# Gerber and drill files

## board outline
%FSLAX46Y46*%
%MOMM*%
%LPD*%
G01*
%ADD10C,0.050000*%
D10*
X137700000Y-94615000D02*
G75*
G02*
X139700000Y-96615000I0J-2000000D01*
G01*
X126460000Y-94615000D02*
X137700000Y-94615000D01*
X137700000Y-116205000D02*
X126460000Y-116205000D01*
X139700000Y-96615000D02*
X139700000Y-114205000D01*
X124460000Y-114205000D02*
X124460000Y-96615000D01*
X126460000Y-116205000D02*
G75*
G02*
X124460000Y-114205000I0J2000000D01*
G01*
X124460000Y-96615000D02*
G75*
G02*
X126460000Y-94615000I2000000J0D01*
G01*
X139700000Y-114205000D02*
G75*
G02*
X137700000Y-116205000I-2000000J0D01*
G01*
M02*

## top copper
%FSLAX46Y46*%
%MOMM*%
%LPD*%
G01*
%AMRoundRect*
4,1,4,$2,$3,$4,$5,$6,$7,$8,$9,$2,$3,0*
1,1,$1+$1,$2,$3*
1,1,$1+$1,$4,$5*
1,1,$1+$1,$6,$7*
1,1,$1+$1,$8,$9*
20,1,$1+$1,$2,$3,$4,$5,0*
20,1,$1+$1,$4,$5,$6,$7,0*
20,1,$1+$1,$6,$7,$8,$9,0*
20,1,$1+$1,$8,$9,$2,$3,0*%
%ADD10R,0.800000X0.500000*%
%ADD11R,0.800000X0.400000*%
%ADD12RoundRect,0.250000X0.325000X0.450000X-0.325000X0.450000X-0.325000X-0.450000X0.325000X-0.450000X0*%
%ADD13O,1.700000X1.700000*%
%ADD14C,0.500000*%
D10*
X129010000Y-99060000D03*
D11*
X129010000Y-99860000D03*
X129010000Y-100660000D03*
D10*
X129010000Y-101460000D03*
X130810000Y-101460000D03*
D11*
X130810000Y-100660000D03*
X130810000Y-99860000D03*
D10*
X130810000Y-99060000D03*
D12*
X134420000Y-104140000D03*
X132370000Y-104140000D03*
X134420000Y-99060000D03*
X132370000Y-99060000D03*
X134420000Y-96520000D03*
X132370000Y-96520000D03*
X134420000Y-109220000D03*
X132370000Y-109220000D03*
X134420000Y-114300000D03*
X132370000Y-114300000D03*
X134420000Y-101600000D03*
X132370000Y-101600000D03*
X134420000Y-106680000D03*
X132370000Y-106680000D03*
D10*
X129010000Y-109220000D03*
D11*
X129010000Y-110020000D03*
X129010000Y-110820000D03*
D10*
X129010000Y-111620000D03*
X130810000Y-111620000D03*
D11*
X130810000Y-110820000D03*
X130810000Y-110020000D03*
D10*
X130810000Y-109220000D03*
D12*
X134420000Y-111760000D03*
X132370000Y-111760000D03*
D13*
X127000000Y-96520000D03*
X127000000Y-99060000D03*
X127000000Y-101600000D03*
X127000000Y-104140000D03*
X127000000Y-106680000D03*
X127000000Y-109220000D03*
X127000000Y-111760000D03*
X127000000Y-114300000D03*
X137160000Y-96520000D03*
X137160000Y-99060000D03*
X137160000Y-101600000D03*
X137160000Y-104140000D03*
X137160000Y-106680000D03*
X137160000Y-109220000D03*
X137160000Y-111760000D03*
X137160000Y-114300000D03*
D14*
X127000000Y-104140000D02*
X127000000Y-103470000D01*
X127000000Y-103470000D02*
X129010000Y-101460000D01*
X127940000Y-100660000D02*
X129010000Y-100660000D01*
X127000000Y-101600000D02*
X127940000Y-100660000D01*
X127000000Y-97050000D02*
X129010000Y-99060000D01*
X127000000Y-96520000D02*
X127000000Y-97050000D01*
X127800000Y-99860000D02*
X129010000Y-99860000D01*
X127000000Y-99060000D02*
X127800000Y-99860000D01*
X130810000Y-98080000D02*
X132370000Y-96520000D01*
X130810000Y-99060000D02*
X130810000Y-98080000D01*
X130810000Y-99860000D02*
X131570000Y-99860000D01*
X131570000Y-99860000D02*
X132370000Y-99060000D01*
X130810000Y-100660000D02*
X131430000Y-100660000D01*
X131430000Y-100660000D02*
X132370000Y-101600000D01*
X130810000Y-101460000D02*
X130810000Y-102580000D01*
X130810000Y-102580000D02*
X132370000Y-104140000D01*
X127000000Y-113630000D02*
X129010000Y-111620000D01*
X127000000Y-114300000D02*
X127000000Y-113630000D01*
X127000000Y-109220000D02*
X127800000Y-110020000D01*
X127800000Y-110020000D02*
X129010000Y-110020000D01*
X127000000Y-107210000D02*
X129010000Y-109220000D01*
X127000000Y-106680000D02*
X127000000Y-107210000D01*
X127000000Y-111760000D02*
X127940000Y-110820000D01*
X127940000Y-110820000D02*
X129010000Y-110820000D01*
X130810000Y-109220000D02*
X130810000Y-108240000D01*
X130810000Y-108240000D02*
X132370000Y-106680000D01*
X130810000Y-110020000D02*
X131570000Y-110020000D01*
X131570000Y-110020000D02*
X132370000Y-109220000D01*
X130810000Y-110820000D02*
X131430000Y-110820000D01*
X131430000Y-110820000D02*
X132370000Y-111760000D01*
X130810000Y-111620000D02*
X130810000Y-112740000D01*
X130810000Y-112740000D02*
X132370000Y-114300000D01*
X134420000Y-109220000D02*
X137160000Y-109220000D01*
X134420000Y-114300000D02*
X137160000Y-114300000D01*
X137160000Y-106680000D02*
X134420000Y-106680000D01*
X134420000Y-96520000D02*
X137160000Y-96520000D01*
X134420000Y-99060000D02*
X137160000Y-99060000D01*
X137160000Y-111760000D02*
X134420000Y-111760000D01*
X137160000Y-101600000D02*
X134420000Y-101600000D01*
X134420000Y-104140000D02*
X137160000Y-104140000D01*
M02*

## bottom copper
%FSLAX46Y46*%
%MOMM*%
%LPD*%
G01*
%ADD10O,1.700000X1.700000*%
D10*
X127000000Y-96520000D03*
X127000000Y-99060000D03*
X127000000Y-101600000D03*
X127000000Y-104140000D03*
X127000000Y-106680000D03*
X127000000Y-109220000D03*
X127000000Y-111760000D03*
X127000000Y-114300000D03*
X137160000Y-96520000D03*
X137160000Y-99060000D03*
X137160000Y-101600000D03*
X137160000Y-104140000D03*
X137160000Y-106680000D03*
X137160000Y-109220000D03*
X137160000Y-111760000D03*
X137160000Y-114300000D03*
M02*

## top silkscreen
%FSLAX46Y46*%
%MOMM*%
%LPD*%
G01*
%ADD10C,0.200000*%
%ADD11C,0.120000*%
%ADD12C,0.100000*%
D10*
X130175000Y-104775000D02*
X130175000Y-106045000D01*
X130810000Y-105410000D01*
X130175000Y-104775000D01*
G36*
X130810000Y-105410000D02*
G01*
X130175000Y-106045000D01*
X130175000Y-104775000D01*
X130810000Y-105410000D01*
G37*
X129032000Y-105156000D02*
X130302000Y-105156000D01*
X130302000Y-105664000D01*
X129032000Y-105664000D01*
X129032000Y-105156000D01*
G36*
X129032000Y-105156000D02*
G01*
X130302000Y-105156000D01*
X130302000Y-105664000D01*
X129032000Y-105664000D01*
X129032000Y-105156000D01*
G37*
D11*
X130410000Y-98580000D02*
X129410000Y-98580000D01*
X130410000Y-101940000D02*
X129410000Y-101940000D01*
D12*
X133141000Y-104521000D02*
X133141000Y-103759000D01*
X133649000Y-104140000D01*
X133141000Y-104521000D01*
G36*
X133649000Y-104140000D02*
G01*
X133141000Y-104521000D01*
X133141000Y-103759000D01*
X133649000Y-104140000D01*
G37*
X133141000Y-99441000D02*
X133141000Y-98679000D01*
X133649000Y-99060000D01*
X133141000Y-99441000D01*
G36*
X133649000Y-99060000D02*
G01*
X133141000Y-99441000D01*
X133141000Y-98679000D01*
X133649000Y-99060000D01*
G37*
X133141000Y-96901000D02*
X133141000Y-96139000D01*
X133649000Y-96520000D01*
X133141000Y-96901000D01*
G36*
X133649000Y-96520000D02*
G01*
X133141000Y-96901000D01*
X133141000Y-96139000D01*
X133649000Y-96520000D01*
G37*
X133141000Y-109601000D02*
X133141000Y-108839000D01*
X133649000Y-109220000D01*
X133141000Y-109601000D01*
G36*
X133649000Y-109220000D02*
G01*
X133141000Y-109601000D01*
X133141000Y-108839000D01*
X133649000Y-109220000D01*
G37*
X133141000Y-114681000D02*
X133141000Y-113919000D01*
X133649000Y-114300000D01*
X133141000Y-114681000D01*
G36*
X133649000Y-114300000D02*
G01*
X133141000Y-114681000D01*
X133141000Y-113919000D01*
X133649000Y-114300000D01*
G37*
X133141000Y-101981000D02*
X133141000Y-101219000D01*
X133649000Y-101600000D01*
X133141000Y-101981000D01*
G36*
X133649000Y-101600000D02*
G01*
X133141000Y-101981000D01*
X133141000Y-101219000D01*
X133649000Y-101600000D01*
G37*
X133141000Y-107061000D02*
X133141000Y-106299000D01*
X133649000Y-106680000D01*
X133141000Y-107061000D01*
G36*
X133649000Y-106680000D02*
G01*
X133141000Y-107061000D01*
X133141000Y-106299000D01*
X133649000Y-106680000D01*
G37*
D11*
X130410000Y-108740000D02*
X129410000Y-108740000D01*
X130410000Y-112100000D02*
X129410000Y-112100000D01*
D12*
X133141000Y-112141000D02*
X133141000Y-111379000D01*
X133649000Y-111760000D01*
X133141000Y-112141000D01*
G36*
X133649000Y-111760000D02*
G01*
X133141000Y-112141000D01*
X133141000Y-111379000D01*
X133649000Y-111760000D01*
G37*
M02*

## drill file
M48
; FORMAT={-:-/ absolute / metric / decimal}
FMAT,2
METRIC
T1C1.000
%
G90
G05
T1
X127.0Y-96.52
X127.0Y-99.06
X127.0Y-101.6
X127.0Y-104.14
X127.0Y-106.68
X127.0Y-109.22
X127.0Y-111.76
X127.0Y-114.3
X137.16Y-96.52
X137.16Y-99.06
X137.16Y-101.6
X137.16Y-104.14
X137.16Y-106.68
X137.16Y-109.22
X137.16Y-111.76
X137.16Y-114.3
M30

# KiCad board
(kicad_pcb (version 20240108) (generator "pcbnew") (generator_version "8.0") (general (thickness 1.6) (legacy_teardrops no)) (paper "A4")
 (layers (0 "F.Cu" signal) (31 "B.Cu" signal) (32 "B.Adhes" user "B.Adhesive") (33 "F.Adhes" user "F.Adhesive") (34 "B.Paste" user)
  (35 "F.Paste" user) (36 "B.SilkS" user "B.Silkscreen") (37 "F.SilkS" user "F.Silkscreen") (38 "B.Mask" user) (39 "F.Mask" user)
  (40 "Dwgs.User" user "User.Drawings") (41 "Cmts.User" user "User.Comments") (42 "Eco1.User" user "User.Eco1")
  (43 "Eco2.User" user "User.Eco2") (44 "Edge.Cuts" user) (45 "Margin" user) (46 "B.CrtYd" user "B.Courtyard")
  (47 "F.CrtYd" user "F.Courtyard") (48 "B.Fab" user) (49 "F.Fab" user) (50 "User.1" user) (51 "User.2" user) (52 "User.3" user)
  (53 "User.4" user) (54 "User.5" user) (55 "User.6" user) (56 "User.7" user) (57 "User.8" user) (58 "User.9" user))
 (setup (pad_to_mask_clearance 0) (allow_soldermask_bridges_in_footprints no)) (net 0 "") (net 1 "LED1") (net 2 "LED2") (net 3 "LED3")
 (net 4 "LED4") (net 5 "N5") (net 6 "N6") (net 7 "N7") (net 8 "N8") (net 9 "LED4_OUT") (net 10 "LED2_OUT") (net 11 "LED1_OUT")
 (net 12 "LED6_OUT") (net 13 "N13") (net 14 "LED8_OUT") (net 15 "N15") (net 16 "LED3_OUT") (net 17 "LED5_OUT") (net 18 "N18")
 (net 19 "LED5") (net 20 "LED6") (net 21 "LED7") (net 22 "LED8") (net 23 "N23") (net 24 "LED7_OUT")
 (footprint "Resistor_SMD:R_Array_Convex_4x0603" (layer "F.Cu") (at 129.91 100.26)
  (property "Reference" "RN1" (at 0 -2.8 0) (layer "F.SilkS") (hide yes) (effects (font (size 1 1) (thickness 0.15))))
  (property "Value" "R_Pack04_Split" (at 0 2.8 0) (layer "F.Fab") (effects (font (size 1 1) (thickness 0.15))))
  (fp_line (start 0.5 -1.68) (end -0.5 -1.68) (stroke (width 0.12) (type solid)) (layer "F.SilkS"))
  (fp_line (start 0.5 1.68) (end -0.5 1.68) (stroke (width 0.12) (type solid)) (layer "F.SilkS"))
  (pad "1" smd rect (at -0.9 -1.2) (size 0.8 0.5) (layers "F.Cu" "F.Paste" "F.Mask") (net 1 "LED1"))
  (pad "2" smd rect (at -0.9 -0.4) (size 0.8 0.4) (layers "F.Cu" "F.Paste" "F.Mask") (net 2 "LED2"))
  (pad "3" smd rect (at -0.9 0.4) (size 0.8 0.4) (layers "F.Cu" "F.Paste" "F.Mask") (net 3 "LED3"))
  (pad "4" smd rect (at -0.9 1.2) (size 0.8 0.5) (layers "F.Cu" "F.Paste" "F.Mask") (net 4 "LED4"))
  (pad "5" smd rect (at 0.9 1.2) (size 0.8 0.5) (layers "F.Cu" "F.Paste" "F.Mask") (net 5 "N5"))
  (pad "6" smd rect (at 0.9 0.4) (size 0.8 0.4) (layers "F.Cu" "F.Paste" "F.Mask") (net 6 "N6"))
  (pad "7" smd rect (at 0.9 -0.4) (size 0.8 0.4) (layers "F.Cu" "F.Paste" "F.Mask") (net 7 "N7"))
  (pad "8" smd rect (at 0.9 -1.2) (size 0.8 0.5) (layers "F.Cu" "F.Paste" "F.Mask") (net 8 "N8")))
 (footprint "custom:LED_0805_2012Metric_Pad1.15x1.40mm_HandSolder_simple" (layer "F.Cu") (at 133.395 104.14 180)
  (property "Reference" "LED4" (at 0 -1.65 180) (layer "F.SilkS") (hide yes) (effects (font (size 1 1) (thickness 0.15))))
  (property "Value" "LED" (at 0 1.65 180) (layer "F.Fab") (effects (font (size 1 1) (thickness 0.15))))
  (fp_poly (pts (xy 0.254 -0.381) (xy 0.254 0.381) (xy -0.254 0)) (stroke (width 0.1) (type solid)) (fill solid) (layer "F.SilkS"))
  (pad "1" smd roundrect (at -1.025 0 180) (size 1.15 1.4) (layers "F.Cu" "F.Paste" "F.Mask") (roundrect_rratio 0.217391) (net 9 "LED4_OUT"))
  (pad "2" smd roundrect (at 1.025 0 180) (size 1.15 1.4) (layers "F.Cu" "F.Paste" "F.Mask") (roundrect_rratio 0.217391) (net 5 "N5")))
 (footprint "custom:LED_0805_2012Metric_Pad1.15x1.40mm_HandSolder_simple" (layer "F.Cu") (at 133.395 99.06 180)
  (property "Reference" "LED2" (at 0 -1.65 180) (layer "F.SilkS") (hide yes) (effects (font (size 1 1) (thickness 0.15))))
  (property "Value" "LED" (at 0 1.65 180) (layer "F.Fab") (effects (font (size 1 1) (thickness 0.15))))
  (fp_poly (pts (xy 0.254 -0.381) (xy 0.254 0.381) (xy -0.254 0)) (stroke (width 0.1) (type solid)) (fill solid) (layer "F.SilkS"))
  (pad "1" smd roundrect (at -1.025 0 180) (size 1.15 1.4) (layers "F.Cu" "F.Paste" "F.Mask") (roundrect_rratio 0.217391)
   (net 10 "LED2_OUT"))
  (pad "2" smd roundrect (at 1.025 0 180) (size 1.15 1.4) (layers "F.Cu" "F.Paste" "F.Mask") (roundrect_rratio 0.217391) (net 7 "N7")))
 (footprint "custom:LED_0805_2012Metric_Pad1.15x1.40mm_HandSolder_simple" (layer "F.Cu") (at 133.395 96.52 180)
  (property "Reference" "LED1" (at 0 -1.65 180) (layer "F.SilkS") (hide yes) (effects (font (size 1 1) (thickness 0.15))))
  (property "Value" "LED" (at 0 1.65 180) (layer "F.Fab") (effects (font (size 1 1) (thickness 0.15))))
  (fp_poly (pts (xy 0.254 -0.381) (xy 0.254 0.381) (xy -0.254 0)) (stroke (width 0.1) (type solid)) (fill solid) (layer "F.SilkS"))
  (pad "1" smd roundrect (at -1.025 0 180) (size 1.15 1.4) (layers "F.Cu" "F.Paste" "F.Mask") (roundrect_rratio 0.217391)
   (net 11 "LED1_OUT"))
  (pad "2" smd roundrect (at 1.025 0 180) (size 1.15 1.4) (layers "F.Cu" "F.Paste" "F.Mask") (roundrect_rratio 0.217391) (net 8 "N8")))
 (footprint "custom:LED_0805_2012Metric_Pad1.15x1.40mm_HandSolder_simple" (layer "F.Cu") (at 133.395 109.22 180)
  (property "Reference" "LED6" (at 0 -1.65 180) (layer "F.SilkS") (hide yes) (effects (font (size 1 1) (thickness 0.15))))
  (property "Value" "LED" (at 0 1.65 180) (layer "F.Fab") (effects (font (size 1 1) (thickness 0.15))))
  (fp_poly (pts (xy 0.254 -0.381) (xy 0.254 0.381) (xy -0.254 0)) (stroke (width 0.1) (type solid)) (fill solid) (layer "F.SilkS"))
  (pad "1" smd roundrect (at -1.025 0 180) (size 1.15 1.4) (layers "F.Cu" "F.Paste" "F.Mask") (roundrect_rratio 0.217391)
   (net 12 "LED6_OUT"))
  (pad "2" smd roundrect (at 1.025 0 180) (size 1.15 1.4) (layers "F.Cu" "F.Paste" "F.Mask") (roundrect_rratio 0.217391) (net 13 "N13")))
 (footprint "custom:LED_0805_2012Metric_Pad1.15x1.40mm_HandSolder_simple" (layer "F.Cu") (at 133.395 114.3 180)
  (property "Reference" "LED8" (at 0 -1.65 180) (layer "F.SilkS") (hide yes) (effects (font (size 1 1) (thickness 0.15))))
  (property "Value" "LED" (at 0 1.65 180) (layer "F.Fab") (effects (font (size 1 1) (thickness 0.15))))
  (fp_poly (pts (xy 0.254 -0.381) (xy 0.254 0.381) (xy -0.254 0)) (stroke (width 0.1) (type solid)) (fill solid) (layer "F.SilkS"))
  (pad "1" smd roundrect (at -1.025 0 180) (size 1.15 1.4) (layers "F.Cu" "F.Paste" "F.Mask") (roundrect_rratio 0.217391)
   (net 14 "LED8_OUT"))
  (pad "2" smd roundrect (at 1.025 0 180) (size 1.15 1.4) (layers "F.Cu" "F.Paste" "F.Mask") (roundrect_rratio 0.217391) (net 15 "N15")))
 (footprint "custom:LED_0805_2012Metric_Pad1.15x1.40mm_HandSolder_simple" (layer "F.Cu") (at 133.395 101.6 180)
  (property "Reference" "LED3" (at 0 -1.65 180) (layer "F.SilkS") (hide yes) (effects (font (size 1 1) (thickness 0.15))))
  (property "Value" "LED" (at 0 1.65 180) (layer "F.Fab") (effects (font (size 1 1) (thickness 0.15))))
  (fp_poly (pts (xy 0.254 -0.381) (xy 0.254 0.381) (xy -0.254 0)) (stroke (width 0.1) (type solid)) (fill solid) (layer "F.SilkS"))
  (pad "1" smd roundrect (at -1.025 0 180) (size 1.15 1.4) (layers "F.Cu" "F.Paste" "F.Mask") (roundrect_rratio 0.217391)
   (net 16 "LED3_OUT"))
  (pad "2" smd roundrect (at 1.025 0 180) (size 1.15 1.4) (layers "F.Cu" "F.Paste" "F.Mask") (roundrect_rratio 0.217391) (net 6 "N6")))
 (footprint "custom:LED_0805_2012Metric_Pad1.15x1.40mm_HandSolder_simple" (layer "F.Cu") (at 133.395 106.68 180)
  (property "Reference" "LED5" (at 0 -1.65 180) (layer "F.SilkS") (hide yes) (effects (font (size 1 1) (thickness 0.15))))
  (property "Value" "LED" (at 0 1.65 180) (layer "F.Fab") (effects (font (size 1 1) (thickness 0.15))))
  (fp_poly (pts (xy 0.254 -0.381) (xy 0.254 0.381) (xy -0.254 0)) (stroke (width 0.1) (type solid)) (fill solid) (layer "F.SilkS"))
  (pad "1" smd roundrect (at -1.025 0 180) (size 1.15 1.4) (layers "F.Cu" "F.Paste" "F.Mask") (roundrect_rratio 0.217391)
   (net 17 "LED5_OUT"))
  (pad "2" smd roundrect (at 1.025 0 180) (size 1.15 1.4) (layers "F.Cu" "F.Paste" "F.Mask") (roundrect_rratio 0.217391) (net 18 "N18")))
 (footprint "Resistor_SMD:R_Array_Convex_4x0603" (layer "F.Cu") (at 129.91 110.42)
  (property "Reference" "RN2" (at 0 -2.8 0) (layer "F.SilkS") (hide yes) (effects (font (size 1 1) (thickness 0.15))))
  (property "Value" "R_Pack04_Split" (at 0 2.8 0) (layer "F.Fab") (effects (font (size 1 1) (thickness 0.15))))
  (fp_line (start 0.5 -1.68) (end -0.5 -1.68) (stroke (width 0.12) (type solid)) (layer "F.SilkS"))
  (fp_line (start 0.5 1.68) (end -0.5 1.68) (stroke (width 0.12) (type solid)) (layer "F.SilkS"))
  (pad "1" smd rect (at -0.9 -1.2) (size 0.8 0.5) (layers "F.Cu" "F.Paste" "F.Mask") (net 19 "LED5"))
  (pad "2" smd rect (at -0.9 -0.4) (size 0.8 0.4) (layers "F.Cu" "F.Paste" "F.Mask") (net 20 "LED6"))
  (pad "3" smd rect (at -0.9 0.4) (size 0.8 0.4) (layers "F.Cu" "F.Paste" "F.Mask") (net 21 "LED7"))
  (pad "4" smd rect (at -0.9 1.2) (size 0.8 0.5) (layers "F.Cu" "F.Paste" "F.Mask") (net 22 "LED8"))
  (pad "5" smd rect (at 0.9 1.2) (size 0.8 0.5) (layers "F.Cu" "F.Paste" "F.Mask") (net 15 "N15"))
  (pad "6" smd rect (at 0.9 0.4) (size 0.8 0.4) (layers "F.Cu" "F.Paste" "F.Mask") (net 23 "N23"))
  (pad "7" smd rect (at 0.9 -0.4) (size 0.8 0.4) (layers "F.Cu" "F.Paste" "F.Mask") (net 13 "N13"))
  (pad "8" smd rect (at 0.9 -1.2) (size 0.8 0.5) (layers "F.Cu" "F.Paste" "F.Mask") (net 18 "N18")))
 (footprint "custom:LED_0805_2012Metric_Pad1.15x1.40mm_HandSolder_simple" (layer "F.Cu") (at 133.395 111.76 180)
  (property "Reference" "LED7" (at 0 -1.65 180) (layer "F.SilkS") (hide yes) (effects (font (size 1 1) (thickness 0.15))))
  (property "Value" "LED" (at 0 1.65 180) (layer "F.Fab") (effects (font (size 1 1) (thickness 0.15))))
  (fp_poly (pts (xy 0.254 -0.381) (xy 0.254 0.381) (xy -0.254 0)) (stroke (width 0.1) (type solid)) (fill solid) (layer "F.SilkS"))
  (pad "1" smd roundrect (at -1.025 0 180) (size 1.15 1.4) (layers "F.Cu" "F.Paste" "F.Mask") (roundrect_rratio 0.217391)
   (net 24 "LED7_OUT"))
  (pad "2" smd roundrect (at 1.025 0 180) (size 1.15 1.4) (layers "F.Cu" "F.Paste" "F.Mask") (roundrect_rratio 0.217391) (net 23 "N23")))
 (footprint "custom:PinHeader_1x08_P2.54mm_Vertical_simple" (layer "B.Cu") (at 127 96.52 180)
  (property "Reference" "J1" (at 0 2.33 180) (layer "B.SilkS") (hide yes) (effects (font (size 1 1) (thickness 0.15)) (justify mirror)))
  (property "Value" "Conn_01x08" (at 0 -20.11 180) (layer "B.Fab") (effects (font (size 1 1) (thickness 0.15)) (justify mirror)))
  (pad "1" thru_hole oval (at 0 0 180) (size 1.7 1.7) (drill 1) (layers "*.Cu" "*.Mask") (remove_unused_layers no) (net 1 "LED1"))
  (pad "2" thru_hole oval (at 0 -2.54 180) (size 1.7 1.7) (drill 1) (layers "*.Cu" "*.Mask") (remove_unused_layers no) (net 2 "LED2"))
  (pad "3" thru_hole oval (at 0 -5.08 180) (size 1.7 1.7) (drill 1) (layers "*.Cu" "*.Mask") (remove_unused_layers no) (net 3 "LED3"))
  (pad "4" thru_hole oval (at 0 -7.62 180) (size 1.7 1.7) (drill 1) (layers "*.Cu" "*.Mask") (remove_unused_layers no) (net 4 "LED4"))
  (pad "5" thru_hole oval (at 0 -10.16 180) (size 1.7 1.7) (drill 1) (layers "*.Cu" "*.Mask") (remove_unused_layers no) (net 19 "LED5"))
  (pad "6" thru_hole oval (at 0 -12.7 180) (size 1.7 1.7) (drill 1) (layers "*.Cu" "*.Mask") (remove_unused_layers no) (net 20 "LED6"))
  (pad "7" thru_hole oval (at 0 -15.24 180) (size 1.7 1.7) (drill 1) (layers "*.Cu" "*.Mask") (remove_unused_layers no) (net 21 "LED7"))
  (pad "8" thru_hole oval (at 0 -17.78 180) (size 1.7 1.7) (drill 1) (layers "*.Cu" "*.Mask") (remove_unused_layers no) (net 22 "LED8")))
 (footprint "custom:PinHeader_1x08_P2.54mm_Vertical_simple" (layer "B.Cu") (at 137.16 96.52 180)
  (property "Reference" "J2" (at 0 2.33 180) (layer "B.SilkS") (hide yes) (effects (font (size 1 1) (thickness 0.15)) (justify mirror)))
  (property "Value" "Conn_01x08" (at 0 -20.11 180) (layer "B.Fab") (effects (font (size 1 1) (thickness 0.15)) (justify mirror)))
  (pad "1" thru_hole oval (at 0 0 180) (size 1.7 1.7) (drill 1) (layers "*.Cu" "*.Mask") (remove_unused_layers no) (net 11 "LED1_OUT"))
  (pad "2" thru_hole oval (at 0 -2.54 180) (size 1.7 1.7) (drill 1) (layers "*.Cu" "*.Mask") (remove_unused_layers no) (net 10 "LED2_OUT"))
  (pad "3" thru_hole oval (at 0 -5.08 180) (size 1.7 1.7) (drill 1) (layers "*.Cu" "*.Mask") (remove_unused_layers no) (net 16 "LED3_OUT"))
  (pad "4" thru_hole oval (at 0 -7.62 180) (size 1.7 1.7) (drill 1) (layers "*.Cu" "*.Mask") (remove_unused_layers no) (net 9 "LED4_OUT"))
  (pad "5" thru_hole oval (at 0 -10.16 180) (size 1.7 1.7) (drill 1) (layers "*.Cu" "*.Mask") (remove_unused_layers no) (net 17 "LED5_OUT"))
  (pad "6" thru_hole oval (at 0 -12.7 180) (size 1.7 1.7) (drill 1) (layers "*.Cu" "*.Mask") (remove_unused_layers no) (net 12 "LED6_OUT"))
  (pad "7" thru_hole oval (at 0 -15.24 180) (size 1.7 1.7) (drill 1) (layers "*.Cu" "*.Mask") (remove_unused_layers no) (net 24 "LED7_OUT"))
  (pad "8" thru_hole oval (at 0 -17.78 180) (size 1.7 1.7) (drill 1) (layers "*.Cu" "*.Mask") (remove_unused_layers no) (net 14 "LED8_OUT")))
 (gr_poly
  (pts (xy 130.175 104.775) (xy 130.175 106.045) (xy 130.81 105.41)) (stroke (width 0.2) (type solid)) (fill solid) (layer "F.SilkS"))
 (gr_rect (start 129.032 105.156) (end 130.302 105.664) (stroke (width 0.2) (type solid)) (fill solid) (layer "F.SilkS"))
 (gr_arc (start 137.7 94.615) (mid 139.114214 95.200786) (end 139.7 96.615) (stroke (width 0.05) (type default)) (layer "Edge.Cuts"))
 (gr_line (start 126.46 94.615) (end 137.7 94.615) (stroke (width 0.05) (type default)) (layer "Edge.Cuts"))
 (gr_line (start 137.7 116.205) (end 126.46 116.205) (stroke (width 0.05) (type default)) (layer "Edge.Cuts"))
 (gr_line (start 139.7 96.615) (end 139.7 114.205) (stroke (width 0.05) (type default)) (layer "Edge.Cuts"))
 (gr_line (start 124.46 114.205) (end 124.46 96.615) (stroke (width 0.05) (type default)) (layer "Edge.Cuts"))
 (gr_arc (start 126.46 116.205) (mid 125.045786 115.619214) (end 124.46 114.205) (stroke (width 0.05) (type default)) (layer "Edge.Cuts"))
 (gr_arc (start 124.46 96.615) (mid 125.045786 95.200786) (end 126.46 94.615) (stroke (width 0.05) (type default)) (layer "Edge.Cuts"))
 (gr_arc (start 139.7 114.205) (mid 139.114214 115.619214) (end 137.7 116.205) (stroke (width 0.05) (type default)) (layer "Edge.Cuts"))
 (segment (start 127 104.14) (end 127 103.47) (width 0.5) (layer "F.Cu") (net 4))
 (segment (start 127 103.47) (end 129.01 101.46) (width 0.5) (layer "F.Cu") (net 4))
 (segment (start 127.94 100.66) (end 129.01 100.66) (width 0.5) (layer "F.Cu") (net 3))
 (segment (start 127 101.6) (end 127.94 100.66) (width 0.5) (layer "F.Cu") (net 3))
 (segment (start 127 97.05) (end 129.01 99.06) (width 0.5) (layer "F.Cu") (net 1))
 (segment (start 127 96.52) (end 127 97.05) (width 0.5) (layer "F.Cu") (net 1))
 (segment (start 127.8 99.86) (end 129.01 99.86) (width 0.5) (layer "F.Cu") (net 2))
 (segment (start 127 99.06) (end 127.8 99.86) (width 0.5) (layer "F.Cu") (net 2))
 (segment (start 130.81 98.08) (end 132.37 96.52) (width 0.5) (layer "F.Cu") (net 8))
 (segment (start 130.81 99.06) (end 130.81 98.08) (width 0.5) (layer "F.Cu") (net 8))
 (segment (start 130.81 99.86) (end 131.57 99.86) (width 0.5) (layer "F.Cu") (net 7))
 (segment (start 131.57 99.86) (end 132.37 99.06) (width 0.5) (layer "F.Cu") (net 7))
 (segment (start 130.81 100.66) (end 131.43 100.66) (width 0.5) (layer "F.Cu") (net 6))
 (segment (start 131.43 100.66) (end 132.37 101.6) (width 0.5) (layer "F.Cu") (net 6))
 (segment (start 130.81 101.46) (end 130.81 102.58) (width 0.5) (layer "F.Cu") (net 5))
 (segment (start 130.81 102.58) (end 132.37 104.14) (width 0.5) (layer "F.Cu") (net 5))
 (segment (start 127 113.63) (end 129.01 111.62) (width 0.5) (layer "F.Cu") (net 22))
 (segment (start 127 114.3) (end 127 113.63) (width 0.5) (layer "F.Cu") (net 22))
 (segment (start 127 109.22) (end 127.8 110.02) (width 0.5) (layer "F.Cu") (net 20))
 (segment (start 127.8 110.02) (end 129.01 110.02) (width 0.5) (layer "F.Cu") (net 20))
 (segment (start 127 107.21) (end 129.01 109.22) (width 0.5) (layer "F.Cu") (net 19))
 (segment (start 127 106.68) (end 127 107.21) (width 0.5) (layer "F.Cu") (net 19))
 (segment (start 127 111.76) (end 127.94 110.82) (width 0.5) (layer "F.Cu") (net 21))
 (segment (start 127.94 110.82) (end 129.01 110.82) (width 0.5) (layer "F.Cu") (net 21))
 (segment (start 130.81 109.22) (end 130.81 108.24) (width 0.5) (layer "F.Cu") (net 18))
 (segment (start 130.81 108.24) (end 132.37 106.68) (width 0.5) (layer "F.Cu") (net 18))
 (segment (start 130.81 110.02) (end 131.57 110.02) (width 0.5) (layer "F.Cu") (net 13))
 (segment (start 131.57 110.02) (end 132.37 109.22) (width 0.5) (layer "F.Cu") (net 13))
 (segment (start 130.81 110.82) (end 131.43 110.82) (width 0.5) (layer "F.Cu") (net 23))
 (segment (start 131.43 110.82) (end 132.37 111.76) (width 0.5) (layer "F.Cu") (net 23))
 (segment (start 130.81 111.62) (end 130.81 112.74) (width 0.5) (layer "F.Cu") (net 15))
 (segment (start 130.81 112.74) (end 132.37 114.3) (width 0.5) (layer "F.Cu") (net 15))
 (segment (start 134.42 109.22) (end 137.16 109.22) (width 0.5) (layer "F.Cu") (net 12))
 (segment (start 134.42 114.3) (end 137.16 114.3) (width 0.5) (layer "F.Cu") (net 14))
 (segment (start 137.16 106.68) (end 134.42 106.68) (width 0.5) (layer "F.Cu") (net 17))
 (segment (start 134.42 96.52) (end 137.16 96.52) (width 0.5) (layer "F.Cu") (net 11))
 (segment (start 134.42 99.06) (end 137.16 99.06) (width 0.5) (layer "F.Cu") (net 10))
 (segment (start 137.16 111.76) (end 134.42 111.76) (width 0.5) (layer "F.Cu") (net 24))
 (segment (start 137.16 101.6) (end 134.42 101.6) (width 0.5) (layer "F.Cu") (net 16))
 (segment (start 134.42 104.14) (end 137.16 104.14) (width 0.5) (layer "F.Cu") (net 9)))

